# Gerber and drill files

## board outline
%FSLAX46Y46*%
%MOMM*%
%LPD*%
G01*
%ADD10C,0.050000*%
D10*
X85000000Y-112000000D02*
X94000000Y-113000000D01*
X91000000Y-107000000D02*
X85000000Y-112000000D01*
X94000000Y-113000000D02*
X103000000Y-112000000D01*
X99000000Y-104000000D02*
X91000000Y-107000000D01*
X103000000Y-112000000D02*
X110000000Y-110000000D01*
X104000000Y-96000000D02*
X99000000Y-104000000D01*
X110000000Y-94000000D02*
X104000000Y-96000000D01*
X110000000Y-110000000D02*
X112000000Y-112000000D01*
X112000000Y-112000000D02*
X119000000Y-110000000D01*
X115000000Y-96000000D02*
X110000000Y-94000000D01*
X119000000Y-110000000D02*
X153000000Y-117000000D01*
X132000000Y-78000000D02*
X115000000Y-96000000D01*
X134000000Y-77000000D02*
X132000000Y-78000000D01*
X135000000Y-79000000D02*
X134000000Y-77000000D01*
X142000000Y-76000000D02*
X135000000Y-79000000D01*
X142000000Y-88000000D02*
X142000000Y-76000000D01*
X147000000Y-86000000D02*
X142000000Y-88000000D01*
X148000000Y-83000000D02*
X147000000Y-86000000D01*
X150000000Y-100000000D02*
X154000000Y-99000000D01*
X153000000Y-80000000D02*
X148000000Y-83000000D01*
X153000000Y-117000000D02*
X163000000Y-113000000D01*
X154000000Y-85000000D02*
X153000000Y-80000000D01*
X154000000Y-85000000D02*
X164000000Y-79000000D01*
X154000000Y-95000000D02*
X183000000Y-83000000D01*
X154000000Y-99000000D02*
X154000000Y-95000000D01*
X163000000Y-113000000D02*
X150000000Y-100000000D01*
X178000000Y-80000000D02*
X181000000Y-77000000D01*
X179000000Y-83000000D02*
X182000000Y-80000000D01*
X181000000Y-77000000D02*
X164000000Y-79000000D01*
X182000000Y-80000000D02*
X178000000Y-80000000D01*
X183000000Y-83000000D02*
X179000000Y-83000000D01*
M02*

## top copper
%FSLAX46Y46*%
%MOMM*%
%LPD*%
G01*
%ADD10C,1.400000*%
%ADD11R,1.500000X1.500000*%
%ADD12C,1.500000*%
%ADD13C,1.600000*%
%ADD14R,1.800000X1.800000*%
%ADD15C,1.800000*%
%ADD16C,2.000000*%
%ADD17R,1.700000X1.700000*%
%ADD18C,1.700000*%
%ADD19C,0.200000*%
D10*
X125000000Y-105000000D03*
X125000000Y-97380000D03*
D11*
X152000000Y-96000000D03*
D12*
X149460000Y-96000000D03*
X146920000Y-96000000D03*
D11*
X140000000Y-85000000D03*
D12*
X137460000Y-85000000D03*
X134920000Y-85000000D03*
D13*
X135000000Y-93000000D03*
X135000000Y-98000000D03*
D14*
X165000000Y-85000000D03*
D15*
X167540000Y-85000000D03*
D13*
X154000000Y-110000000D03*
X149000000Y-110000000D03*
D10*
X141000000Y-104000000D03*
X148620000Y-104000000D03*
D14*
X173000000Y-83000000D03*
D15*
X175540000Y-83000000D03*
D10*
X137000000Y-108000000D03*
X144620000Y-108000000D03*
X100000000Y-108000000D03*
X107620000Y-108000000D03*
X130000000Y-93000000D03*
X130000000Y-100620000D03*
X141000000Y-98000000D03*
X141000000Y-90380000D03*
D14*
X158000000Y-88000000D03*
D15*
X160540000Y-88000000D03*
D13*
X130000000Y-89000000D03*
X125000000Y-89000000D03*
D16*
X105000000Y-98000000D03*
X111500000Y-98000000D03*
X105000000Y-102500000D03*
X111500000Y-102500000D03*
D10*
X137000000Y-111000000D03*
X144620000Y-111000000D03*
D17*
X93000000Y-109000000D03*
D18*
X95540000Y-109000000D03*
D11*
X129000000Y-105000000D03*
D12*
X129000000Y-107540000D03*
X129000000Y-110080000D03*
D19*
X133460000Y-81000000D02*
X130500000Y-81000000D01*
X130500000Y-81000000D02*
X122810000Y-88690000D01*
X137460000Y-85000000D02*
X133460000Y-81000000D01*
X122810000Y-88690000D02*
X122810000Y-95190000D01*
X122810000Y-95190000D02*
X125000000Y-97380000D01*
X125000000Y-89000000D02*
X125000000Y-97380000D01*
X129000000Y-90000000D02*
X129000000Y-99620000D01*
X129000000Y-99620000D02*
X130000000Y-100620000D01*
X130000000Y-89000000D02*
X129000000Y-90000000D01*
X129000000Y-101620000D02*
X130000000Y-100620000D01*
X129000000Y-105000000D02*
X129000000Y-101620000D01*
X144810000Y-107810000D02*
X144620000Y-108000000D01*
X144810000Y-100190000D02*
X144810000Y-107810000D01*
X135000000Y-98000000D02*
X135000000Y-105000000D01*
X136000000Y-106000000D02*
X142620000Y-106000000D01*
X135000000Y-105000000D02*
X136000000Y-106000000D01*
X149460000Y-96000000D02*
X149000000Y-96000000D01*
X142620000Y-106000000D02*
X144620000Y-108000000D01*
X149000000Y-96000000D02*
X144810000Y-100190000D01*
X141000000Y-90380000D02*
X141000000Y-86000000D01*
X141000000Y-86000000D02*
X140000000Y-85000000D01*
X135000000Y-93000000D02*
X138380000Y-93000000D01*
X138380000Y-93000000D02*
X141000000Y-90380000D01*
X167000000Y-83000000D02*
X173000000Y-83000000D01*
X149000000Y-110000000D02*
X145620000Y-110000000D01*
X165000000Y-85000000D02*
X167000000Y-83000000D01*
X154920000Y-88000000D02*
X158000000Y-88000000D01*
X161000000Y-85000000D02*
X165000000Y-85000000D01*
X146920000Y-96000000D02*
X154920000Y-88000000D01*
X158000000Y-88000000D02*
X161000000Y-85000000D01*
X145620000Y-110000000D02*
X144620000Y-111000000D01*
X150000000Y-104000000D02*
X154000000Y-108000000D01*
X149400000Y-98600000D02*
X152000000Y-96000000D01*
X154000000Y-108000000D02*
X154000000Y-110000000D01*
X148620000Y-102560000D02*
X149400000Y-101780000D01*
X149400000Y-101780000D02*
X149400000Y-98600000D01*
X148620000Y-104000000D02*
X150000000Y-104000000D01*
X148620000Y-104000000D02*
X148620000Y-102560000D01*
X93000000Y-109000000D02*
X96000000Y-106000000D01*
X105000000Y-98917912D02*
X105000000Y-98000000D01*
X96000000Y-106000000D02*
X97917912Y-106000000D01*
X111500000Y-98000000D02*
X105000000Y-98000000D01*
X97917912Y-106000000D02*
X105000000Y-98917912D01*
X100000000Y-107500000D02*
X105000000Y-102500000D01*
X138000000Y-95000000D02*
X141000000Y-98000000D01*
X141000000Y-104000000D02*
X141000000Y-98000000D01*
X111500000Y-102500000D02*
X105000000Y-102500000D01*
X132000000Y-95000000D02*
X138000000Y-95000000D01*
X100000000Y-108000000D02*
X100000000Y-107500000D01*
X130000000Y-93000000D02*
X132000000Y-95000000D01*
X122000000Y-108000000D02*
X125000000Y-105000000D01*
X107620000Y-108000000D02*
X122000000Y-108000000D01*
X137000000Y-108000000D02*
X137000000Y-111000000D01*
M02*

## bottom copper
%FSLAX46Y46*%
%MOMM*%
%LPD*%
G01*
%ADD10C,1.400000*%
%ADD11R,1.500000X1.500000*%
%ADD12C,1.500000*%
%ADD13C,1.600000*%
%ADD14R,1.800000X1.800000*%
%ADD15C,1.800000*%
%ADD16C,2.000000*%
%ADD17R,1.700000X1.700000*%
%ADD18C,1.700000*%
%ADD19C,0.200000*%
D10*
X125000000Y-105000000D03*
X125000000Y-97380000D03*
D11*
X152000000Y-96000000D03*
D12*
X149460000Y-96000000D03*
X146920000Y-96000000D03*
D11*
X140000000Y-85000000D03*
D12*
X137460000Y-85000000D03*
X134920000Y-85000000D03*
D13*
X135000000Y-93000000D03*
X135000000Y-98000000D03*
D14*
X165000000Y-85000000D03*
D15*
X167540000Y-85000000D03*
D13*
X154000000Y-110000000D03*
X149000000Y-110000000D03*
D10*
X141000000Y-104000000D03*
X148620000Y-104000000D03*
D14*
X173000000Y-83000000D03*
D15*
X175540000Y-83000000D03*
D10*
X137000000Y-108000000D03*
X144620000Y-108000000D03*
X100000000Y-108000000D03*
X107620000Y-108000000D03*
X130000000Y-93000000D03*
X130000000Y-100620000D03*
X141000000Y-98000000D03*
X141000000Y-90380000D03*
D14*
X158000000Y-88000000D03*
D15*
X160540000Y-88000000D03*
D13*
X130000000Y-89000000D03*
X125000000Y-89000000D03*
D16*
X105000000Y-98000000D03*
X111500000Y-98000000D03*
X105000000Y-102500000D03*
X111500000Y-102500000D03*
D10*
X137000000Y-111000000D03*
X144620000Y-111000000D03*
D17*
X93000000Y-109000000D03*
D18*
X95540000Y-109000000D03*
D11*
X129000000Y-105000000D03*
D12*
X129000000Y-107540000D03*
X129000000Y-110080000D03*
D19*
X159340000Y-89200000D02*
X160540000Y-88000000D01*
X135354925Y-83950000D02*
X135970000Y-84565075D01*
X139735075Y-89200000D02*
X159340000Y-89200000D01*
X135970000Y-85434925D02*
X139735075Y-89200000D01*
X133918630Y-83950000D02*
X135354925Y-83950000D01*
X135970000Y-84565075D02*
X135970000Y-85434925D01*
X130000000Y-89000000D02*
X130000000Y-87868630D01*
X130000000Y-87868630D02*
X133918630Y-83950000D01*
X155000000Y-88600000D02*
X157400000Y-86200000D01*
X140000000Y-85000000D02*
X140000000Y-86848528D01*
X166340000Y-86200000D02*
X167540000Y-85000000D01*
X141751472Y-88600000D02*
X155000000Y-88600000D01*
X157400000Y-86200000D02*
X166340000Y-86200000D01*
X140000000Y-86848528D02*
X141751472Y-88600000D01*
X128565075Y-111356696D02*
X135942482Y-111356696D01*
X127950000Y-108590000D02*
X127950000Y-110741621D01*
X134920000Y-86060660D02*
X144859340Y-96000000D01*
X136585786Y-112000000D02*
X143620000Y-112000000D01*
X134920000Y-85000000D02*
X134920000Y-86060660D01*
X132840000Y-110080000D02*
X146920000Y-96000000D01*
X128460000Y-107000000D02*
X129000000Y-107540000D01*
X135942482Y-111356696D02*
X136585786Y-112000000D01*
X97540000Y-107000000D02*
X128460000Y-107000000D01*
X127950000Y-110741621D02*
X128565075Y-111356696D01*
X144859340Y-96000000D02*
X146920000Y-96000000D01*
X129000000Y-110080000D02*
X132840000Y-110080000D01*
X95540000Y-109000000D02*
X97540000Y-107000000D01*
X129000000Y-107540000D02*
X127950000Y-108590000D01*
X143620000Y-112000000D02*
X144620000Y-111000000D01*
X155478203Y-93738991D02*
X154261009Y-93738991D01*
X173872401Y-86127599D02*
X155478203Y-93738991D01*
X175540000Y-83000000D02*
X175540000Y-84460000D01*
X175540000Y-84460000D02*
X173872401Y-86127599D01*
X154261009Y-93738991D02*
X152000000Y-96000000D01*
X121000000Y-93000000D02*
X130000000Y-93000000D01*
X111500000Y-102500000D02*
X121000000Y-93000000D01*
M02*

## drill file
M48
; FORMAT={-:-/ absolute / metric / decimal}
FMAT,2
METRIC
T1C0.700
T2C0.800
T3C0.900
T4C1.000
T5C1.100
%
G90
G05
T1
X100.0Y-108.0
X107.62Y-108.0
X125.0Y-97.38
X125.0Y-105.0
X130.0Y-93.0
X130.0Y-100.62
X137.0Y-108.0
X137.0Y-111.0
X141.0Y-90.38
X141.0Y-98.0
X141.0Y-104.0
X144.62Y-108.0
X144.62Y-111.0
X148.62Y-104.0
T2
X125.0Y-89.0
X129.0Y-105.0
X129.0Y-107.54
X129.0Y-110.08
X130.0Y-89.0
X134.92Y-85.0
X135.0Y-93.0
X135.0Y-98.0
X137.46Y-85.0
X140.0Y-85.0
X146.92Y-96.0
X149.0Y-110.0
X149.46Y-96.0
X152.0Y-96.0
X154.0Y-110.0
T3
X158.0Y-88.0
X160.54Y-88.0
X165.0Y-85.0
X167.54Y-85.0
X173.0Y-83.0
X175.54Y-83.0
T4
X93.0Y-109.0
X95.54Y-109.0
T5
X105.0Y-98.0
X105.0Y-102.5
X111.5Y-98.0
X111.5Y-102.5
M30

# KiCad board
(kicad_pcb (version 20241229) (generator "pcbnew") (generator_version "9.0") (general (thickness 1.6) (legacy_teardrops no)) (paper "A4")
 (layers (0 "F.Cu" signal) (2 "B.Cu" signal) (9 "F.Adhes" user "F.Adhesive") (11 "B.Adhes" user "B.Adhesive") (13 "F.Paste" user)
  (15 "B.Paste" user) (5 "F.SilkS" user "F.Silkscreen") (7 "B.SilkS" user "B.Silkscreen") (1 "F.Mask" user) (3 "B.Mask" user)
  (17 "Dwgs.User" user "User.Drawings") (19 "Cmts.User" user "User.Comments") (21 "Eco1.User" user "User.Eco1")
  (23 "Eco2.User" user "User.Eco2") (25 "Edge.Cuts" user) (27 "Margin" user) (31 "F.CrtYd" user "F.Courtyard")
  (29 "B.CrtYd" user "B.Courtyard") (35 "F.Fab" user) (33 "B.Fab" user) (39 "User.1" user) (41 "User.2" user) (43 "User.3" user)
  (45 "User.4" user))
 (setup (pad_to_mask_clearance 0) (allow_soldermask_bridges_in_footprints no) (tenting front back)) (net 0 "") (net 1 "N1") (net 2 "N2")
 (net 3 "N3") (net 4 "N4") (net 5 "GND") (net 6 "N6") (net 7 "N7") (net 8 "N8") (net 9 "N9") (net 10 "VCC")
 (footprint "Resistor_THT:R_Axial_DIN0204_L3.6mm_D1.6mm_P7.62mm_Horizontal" (layer "F.Cu") (at 125 105 90)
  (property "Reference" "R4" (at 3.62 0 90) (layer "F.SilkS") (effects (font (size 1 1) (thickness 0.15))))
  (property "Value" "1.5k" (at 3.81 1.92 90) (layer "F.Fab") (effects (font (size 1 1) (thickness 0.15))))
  (pad "1" thru_hole circle (at 0 0 90) (size 1.4 1.4) (drill 0.7) (layers "*.Cu" "*.Mask") (remove_unused_layers no) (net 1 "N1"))
  (pad "2" thru_hole circle (at 7.62 0 90) (size 1.4 1.4) (drill 0.7) (layers "*.Cu" "*.Mask") (remove_unused_layers no) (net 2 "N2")))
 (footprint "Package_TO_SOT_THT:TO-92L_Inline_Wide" (layer "F.Cu") (at 152 96 180)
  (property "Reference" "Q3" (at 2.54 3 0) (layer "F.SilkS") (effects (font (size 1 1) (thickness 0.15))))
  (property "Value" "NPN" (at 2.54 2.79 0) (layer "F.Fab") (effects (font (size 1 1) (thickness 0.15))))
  (pad "1" thru_hole rect (at 0 0 180) (size 1.5 1.5) (drill 0.8) (layers "*.Cu" "*.Mask") (remove_unused_layers no) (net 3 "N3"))
  (pad "2" thru_hole circle (at 2.54 0 180) (size 1.5 1.5) (drill 0.8) (layers "*.Cu" "*.Mask") (remove_unused_layers no) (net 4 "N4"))
  (pad "3" thru_hole circle (at 5.08 0 180) (size 1.5 1.5) (drill 0.8) (layers "*.Cu" "*.Mask") (remove_unused_layers no) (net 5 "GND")))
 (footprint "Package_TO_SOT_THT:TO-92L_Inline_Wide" (layer "F.Cu") (at 140 85 180)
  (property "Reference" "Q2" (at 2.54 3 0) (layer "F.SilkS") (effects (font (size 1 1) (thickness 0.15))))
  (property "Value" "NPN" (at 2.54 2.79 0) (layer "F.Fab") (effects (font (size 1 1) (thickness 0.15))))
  (pad "1" thru_hole rect (at 0 0 180) (size 1.5 1.5) (drill 0.8) (layers "*.Cu" "*.Mask") (remove_unused_layers no) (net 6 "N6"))
  (pad "2" thru_hole circle (at 2.54 0 180) (size 1.5 1.5) (drill 0.8) (layers "*.Cu" "*.Mask") (remove_unused_layers no) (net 2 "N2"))
  (pad "3" thru_hole circle (at 5.08 0 180) (size 1.5 1.5) (drill 0.8) (layers "*.Cu" "*.Mask") (remove_unused_layers no) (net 5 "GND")))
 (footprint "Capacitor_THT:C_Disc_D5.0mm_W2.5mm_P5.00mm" (layer "F.Cu") (at 135 93 -90)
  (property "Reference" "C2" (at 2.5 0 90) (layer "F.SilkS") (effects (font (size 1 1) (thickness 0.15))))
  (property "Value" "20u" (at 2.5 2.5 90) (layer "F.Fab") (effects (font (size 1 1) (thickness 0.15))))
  (pad "1" thru_hole circle (at 0 0 270) (size 1.6 1.6) (drill 0.8) (layers "*.Cu" "*.Mask") (remove_unused_layers no) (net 6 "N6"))
  (pad "2" thru_hole circle (at 5 0 270) (size 1.6 1.6) (drill 0.8) (layers "*.Cu" "*.Mask") (remove_unused_layers no) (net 4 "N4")))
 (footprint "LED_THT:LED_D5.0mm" (layer "F.Cu") (at 165 85)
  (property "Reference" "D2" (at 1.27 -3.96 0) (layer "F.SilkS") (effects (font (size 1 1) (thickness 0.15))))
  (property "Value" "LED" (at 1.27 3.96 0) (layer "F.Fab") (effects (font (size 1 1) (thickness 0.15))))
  (pad "1" thru_hole rect (at 0 0) (size 1.8 1.8) (drill 0.9) (layers "*.Cu" "*.Mask") (remove_unused_layers no) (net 5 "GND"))
  (pad "2" thru_hole circle (at 2.54 0) (size 1.8 1.8) (drill 0.9) (layers "*.Cu" "*.Mask") (remove_unused_layers no) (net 6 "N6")))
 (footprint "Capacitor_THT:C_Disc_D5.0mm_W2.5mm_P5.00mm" (layer "F.Cu") (at 154 110 180)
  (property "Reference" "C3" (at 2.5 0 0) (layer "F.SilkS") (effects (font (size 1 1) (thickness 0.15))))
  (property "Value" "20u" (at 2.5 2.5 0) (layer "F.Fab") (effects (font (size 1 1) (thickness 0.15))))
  (pad "1" thru_hole circle (at 0 0 180) (size 1.6 1.6) (drill 0.8) (layers "*.Cu" "*.Mask") (remove_unused_layers no) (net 3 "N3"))
  (pad "2" thru_hole circle (at 5 0 180) (size 1.6 1.6) (drill 0.8) (layers "*.Cu" "*.Mask") (remove_unused_layers no) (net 5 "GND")))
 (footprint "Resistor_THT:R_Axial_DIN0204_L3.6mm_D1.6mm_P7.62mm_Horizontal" (layer "F.Cu") (at 141 104)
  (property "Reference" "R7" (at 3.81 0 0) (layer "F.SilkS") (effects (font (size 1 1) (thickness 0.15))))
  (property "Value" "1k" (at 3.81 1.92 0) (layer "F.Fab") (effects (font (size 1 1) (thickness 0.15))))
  (pad "1" thru_hole circle (at 0 0) (size 1.4 1.4) (drill 0.7) (layers "*.Cu" "*.Mask") (remove_unused_layers no) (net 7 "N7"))
  (pad "2" thru_hole circle (at 7.62 0) (size 1.4 1.4) (drill 0.7) (layers "*.Cu" "*.Mask") (remove_unused_layers no) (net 3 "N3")))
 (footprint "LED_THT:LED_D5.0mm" (layer "F.Cu") (at 173 83)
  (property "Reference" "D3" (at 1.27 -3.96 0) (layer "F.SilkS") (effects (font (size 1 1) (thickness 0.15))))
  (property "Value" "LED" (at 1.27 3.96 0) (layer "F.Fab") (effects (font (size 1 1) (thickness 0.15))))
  (pad "1" thru_hole rect (at 0 0) (size 1.8 1.8) (drill 0.9) (layers "*.Cu" "*.Mask") (remove_unused_layers no) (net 5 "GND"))
  (pad "2" thru_hole circle (at 2.54 0) (size 1.8 1.8) (drill 0.9) (layers "*.Cu" "*.Mask") (remove_unused_layers no) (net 3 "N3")))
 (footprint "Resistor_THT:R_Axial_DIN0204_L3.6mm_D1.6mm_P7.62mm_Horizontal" (layer "F.Cu") (at 137 108)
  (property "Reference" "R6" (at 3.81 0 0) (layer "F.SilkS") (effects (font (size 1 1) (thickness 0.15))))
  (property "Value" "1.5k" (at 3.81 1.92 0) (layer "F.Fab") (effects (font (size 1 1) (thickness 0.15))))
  (pad "1" thru_hole circle (at 0 0) (size 1.4 1.4) (drill 0.7) (layers "*.Cu" "*.Mask") (remove_unused_layers no) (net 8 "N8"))
  (pad "2" thru_hole circle (at 7.62 0) (size 1.4 1.4) (drill 0.7) (layers "*.Cu" "*.Mask") (remove_unused_layers no) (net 4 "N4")))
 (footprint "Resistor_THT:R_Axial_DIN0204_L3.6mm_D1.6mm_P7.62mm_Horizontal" (layer "F.Cu") (at 100 108)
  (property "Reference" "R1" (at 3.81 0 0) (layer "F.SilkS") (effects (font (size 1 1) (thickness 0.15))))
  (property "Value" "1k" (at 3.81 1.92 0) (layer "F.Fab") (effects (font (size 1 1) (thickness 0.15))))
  (pad "1" thru_hole circle (at 0 0) (size 1.4 1.4) (drill 0.7) (layers "*.Cu" "*.Mask") (remove_unused_layers no) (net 7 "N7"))
  (pad "2" thru_hole circle (at 7.62 0) (size 1.4 1.4) (drill 0.7) (layers "*.Cu" "*.Mask") (remove_unused_layers no) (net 1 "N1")))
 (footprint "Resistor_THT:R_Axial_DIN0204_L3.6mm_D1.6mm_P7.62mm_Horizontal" (layer "F.Cu") (at 130 93 -90)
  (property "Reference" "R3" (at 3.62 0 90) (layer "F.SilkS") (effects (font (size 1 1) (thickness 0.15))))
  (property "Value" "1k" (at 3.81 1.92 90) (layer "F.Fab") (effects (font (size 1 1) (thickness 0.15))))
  (pad "1" thru_hole circle (at 0 0 270) (size 1.4 1.4) (drill 0.7) (layers "*.Cu" "*.Mask") (remove_unused_layers no) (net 7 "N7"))
  (pad "2" thru_hole circle (at 7.62 0 270) (size 1.4 1.4) (drill 0.7) (layers "*.Cu" "*.Mask") (remove_unused_layers no) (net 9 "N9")))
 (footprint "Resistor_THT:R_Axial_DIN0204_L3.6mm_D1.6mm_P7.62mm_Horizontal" (layer "F.Cu") (at 141 98 90)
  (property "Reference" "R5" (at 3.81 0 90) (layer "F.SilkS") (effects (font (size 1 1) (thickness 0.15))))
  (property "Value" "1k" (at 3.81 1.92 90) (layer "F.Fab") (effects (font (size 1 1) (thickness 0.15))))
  (pad "1" thru_hole circle (at 0 0 90) (size 1.4 1.4) (drill 0.7) (layers "*.Cu" "*.Mask") (remove_unused_layers no) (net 7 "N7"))
  (pad "2" thru_hole circle (at 7.62 0 90) (size 1.4 1.4) (drill 0.7) (layers "*.Cu" "*.Mask") (remove_unused_layers no) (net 6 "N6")))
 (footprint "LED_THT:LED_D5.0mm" (layer "F.Cu") (at 158 88)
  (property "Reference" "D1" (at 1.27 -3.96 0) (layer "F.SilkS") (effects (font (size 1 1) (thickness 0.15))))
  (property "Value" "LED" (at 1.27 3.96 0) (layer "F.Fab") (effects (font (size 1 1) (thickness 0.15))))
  (pad "1" thru_hole rect (at 0 0) (size 1.8 1.8) (drill 0.9) (layers "*.Cu" "*.Mask") (remove_unused_layers no) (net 5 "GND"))
  (pad "2" thru_hole circle (at 2.54 0) (size 1.8 1.8) (drill 0.9) (layers "*.Cu" "*.Mask") (remove_unused_layers no) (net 9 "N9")))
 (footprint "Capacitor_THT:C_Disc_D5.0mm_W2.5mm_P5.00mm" (layer "F.Cu") (at 130 89 180)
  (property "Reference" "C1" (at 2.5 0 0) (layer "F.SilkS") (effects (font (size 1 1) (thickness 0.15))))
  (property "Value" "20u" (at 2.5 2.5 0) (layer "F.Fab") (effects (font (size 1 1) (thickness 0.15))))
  (pad "1" thru_hole circle (at 0 0 180) (size 1.6 1.6) (drill 0.8) (layers "*.Cu" "*.Mask") (remove_unused_layers no) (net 9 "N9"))
  (pad "2" thru_hole circle (at 5 0 180) (size 1.6 1.6) (drill 0.8) (layers "*.Cu" "*.Mask") (remove_unused_layers no) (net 2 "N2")))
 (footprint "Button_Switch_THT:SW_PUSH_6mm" (layer "F.Cu") (at 105 98)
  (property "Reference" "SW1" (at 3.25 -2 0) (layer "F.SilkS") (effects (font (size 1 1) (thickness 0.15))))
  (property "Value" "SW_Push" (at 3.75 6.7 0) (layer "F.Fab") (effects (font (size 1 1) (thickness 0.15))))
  (pad "1" thru_hole circle (at 0 0 90) (size 2 2) (drill 1.1) (layers "*.Cu" "*.Mask") (remove_unused_layers no) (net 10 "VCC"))
  (pad "1" thru_hole circle (at 6.5 0 90) (size 2 2) (drill 1.1) (layers "*.Cu" "*.Mask") (remove_unused_layers no) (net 10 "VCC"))
  (pad "2" thru_hole circle (at 0 4.5 90) (size 2 2) (drill 1.1) (layers "*.Cu" "*.Mask") (remove_unused_layers no) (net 7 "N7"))
  (pad "2" thru_hole circle (at 6.5 4.5 90) (size 2 2) (drill 1.1) (layers "*.Cu" "*.Mask") (remove_unused_layers no) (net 7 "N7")))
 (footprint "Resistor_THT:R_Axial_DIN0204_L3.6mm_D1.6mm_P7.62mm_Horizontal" (layer "F.Cu") (at 137 111)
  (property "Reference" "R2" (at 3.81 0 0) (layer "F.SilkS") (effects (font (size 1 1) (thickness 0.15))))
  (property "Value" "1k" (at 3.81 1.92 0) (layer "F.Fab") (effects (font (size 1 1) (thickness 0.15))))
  (pad "1" thru_hole circle (at 0 0) (size 1.4 1.4) (drill 0.7) (layers "*.Cu" "*.Mask") (remove_unused_layers no) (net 8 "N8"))
  (pad "2" thru_hole circle (at 7.62 0) (size 1.4 1.4) (drill 0.7) (layers "*.Cu" "*.Mask") (remove_unused_layers no) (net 5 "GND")))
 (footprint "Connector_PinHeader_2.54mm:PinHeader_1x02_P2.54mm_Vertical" (layer "F.Cu") (at 93 109 90)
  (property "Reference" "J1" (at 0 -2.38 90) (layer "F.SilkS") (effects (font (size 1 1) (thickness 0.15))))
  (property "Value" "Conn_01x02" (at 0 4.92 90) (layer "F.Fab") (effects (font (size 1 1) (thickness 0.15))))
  (pad "1" thru_hole rect (at 0 0 90) (size 1.7 1.7) (drill 1) (layers "*.Cu" "*.Mask") (remove_unused_layers no) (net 10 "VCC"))
  (pad "2" thru_hole circle (at 0 2.54 90) (size 1.7 1.7) (drill 1) (layers "*.Cu" "*.Mask") (remove_unused_layers no) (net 5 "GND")))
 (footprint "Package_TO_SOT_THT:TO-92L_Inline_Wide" (layer "F.Cu") (at 129 105 -90)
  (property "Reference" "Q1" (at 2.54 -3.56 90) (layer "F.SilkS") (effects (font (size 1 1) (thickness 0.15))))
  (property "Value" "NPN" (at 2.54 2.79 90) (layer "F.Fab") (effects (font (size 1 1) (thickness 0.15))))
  (pad "1" thru_hole rect (at 0 0 270) (size 1.5 1.5) (drill 0.8) (layers "*.Cu" "*.Mask") (remove_unused_layers no) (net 9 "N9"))
  (pad "2" thru_hole circle (at 2.54 0 270) (size 1.5 1.5) (drill 0.8) (layers "*.Cu" "*.Mask") (remove_unused_layers no) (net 5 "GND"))
  (pad "3" thru_hole circle (at 5.08 0 270) (size 1.5 1.5) (drill 0.8) (layers "*.Cu" "*.Mask") (remove_unused_layers no) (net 5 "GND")))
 (gr_line (start 85 112) (end 94 113) (stroke (width 0.05) (type default)) (layer "Edge.Cuts"))
 (gr_line (start 91 107) (end 85 112) (stroke (width 0.05) (type default)) (layer "Edge.Cuts"))
 (gr_line (start 94 113) (end 103 112) (stroke (width 0.05) (type default)) (layer "Edge.Cuts"))
 (gr_line (start 99 104) (end 91 107) (stroke (width 0.05) (type default)) (layer "Edge.Cuts"))
 (gr_line (start 103 112) (end 110 110) (stroke (width 0.05) (type default)) (layer "Edge.Cuts"))
 (gr_line (start 104 96) (end 99 104) (stroke (width 0.05) (type default)) (layer "Edge.Cuts"))
 (gr_line (start 110 94) (end 104 96) (stroke (width 0.05) (type default)) (layer "Edge.Cuts"))
 (gr_line (start 110 110) (end 112 112) (stroke (width 0.05) (type default)) (layer "Edge.Cuts"))
 (gr_line (start 112 112) (end 119 110) (stroke (width 0.05) (type default)) (layer "Edge.Cuts"))
 (gr_line (start 115 96) (end 110 94) (stroke (width 0.05) (type default)) (layer "Edge.Cuts"))
 (gr_line (start 119 110) (end 153 117) (stroke (width 0.05) (type default)) (layer "Edge.Cuts"))
 (gr_line (start 132 78) (end 115 96) (stroke (width 0.05) (type default)) (layer "Edge.Cuts"))
 (gr_line (start 134 77) (end 132 78) (stroke (width 0.05) (type default)) (layer "Edge.Cuts"))
 (gr_line (start 135 79) (end 134 77) (stroke (width 0.05) (type default)) (layer "Edge.Cuts"))
 (gr_line (start 142 76) (end 135 79) (stroke (width 0.05) (type default)) (layer "Edge.Cuts"))
 (gr_line (start 142 88) (end 142 76) (stroke (width 0.05) (type default)) (layer "Edge.Cuts"))
 (gr_line (start 147 86) (end 142 88) (stroke (width 0.05) (type default)) (layer "Edge.Cuts"))
 (gr_line (start 148 83) (end 147 86) (stroke (width 0.05) (type default)) (layer "Edge.Cuts"))
 (gr_line (start 150 100) (end 154 99) (stroke (width 0.05) (type default)) (layer "Edge.Cuts"))
 (gr_line (start 153 80) (end 148 83) (stroke (width 0.05) (type default)) (layer "Edge.Cuts"))
 (gr_line (start 153 117) (end 163 113) (stroke (width 0.05) (type default)) (layer "Edge.Cuts"))
 (gr_line (start 154 85) (end 153 80) (stroke (width 0.05) (type default)) (layer "Edge.Cuts"))
 (gr_line (start 154 85) (end 164 79) (stroke (width 0.05) (type default)) (layer "Edge.Cuts"))
 (gr_line (start 154 95) (end 183 83) (stroke (width 0.05) (type default)) (layer "Edge.Cuts"))
 (gr_line (start 154 99) (end 154 95) (stroke (width 0.05) (type default)) (layer "Edge.Cuts"))
 (gr_line (start 163 113) (end 150 100) (stroke (width 0.05) (type default)) (layer "Edge.Cuts"))
 (gr_line (start 178 80) (end 181 77) (stroke (width 0.05) (type default)) (layer "Edge.Cuts"))
 (gr_line (start 179 83) (end 182 80) (stroke (width 0.05) (type default)) (layer "Edge.Cuts"))
 (gr_line (start 181 77) (end 164 79) (stroke (width 0.05) (type default)) (layer "Edge.Cuts"))
 (gr_line (start 182 80) (end 178 80) (stroke (width 0.05) (type default)) (layer "Edge.Cuts"))
 (gr_line (start 183 83) (end 179 83) (stroke (width 0.05) (type default)) (layer "Edge.Cuts"))
 (segment (start 133.46 81) (end 130.5 81) (width 0.2) (layer "F.Cu") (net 2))
 (segment (start 130.5 81) (end 122.81 88.69) (width 0.2) (layer "F.Cu") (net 2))
 (segment (start 137.46 85) (end 133.46 81) (width 0.2) (layer "F.Cu") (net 2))
 (segment (start 122.81 88.69) (end 122.81 95.19) (width 0.2) (layer "F.Cu") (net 2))
 (segment (start 122.81 95.19) (end 125 97.38) (width 0.2) (layer "F.Cu") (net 2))
 (segment (start 125 89) (end 125 97.38) (width 0.2) (layer "F.Cu") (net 2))
 (segment (start 129 90) (end 129 99.62) (width 0.2) (layer "F.Cu") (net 9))
 (segment (start 129 99.62) (end 130 100.62) (width 0.2) (layer "F.Cu") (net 9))
 (segment (start 130 89) (end 129 90) (width 0.2) (layer "F.Cu") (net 9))
 (segment (start 129 101.62) (end 130 100.62) (width 0.2) (layer "F.Cu") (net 9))
 (segment (start 129 105) (end 129 101.62) (width 0.2) (layer "F.Cu") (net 9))
 (segment (start 159.34 89.2) (end 160.54 88) (width 0.2) (layer "B.Cu") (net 9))
 (segment (start 135.354925 83.95) (end 135.97 84.565075) (width 0.2) (layer "B.Cu") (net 9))
 (segment (start 139.735075 89.2) (end 159.34 89.2) (width 0.2) (layer "B.Cu") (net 9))
 (segment (start 135.97 85.434925) (end 139.735075 89.2) (width 0.2) (layer "B.Cu") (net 9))
 (segment (start 133.91863 83.95) (end 135.354925 83.95) (width 0.2) (layer "B.Cu") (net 9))
 (segment (start 135.97 84.565075) (end 135.97 85.434925) (width 0.2) (layer "B.Cu") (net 9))
 (segment (start 130 89) (end 130 87.86863) (width 0.2) (layer "B.Cu") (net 9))
 (segment (start 130 87.86863) (end 133.91863 83.95) (width 0.2) (layer "B.Cu") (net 9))
 (segment (start 144.81 107.81) (end 144.62 108) (width 0.2) (layer "F.Cu") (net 4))
 (segment (start 144.81 100.19) (end 144.81 107.81) (width 0.2) (layer "F.Cu") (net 4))
 (segment (start 135 98) (end 135 105) (width 0.2) (layer "F.Cu") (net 4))
 (segment (start 136 106) (end 142.62 106) (width 0.2) (layer "F.Cu") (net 4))
 (segment (start 135 105) (end 136 106) (width 0.2) (layer "F.Cu") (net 4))
 (segment (start 149.46 96) (end 149 96) (width 0.2) (layer "F.Cu") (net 4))
 (segment (start 142.62 106) (end 144.62 108) (width 0.2) (layer "F.Cu") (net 4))
 (segment (start 149 96) (end 144.81 100.19) (width 0.2) (layer "F.Cu") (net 4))
 (segment (start 141 90.38) (end 141 86) (width 0.2) (layer "F.Cu") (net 6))
 (segment (start 141 86) (end 140 85) (width 0.2) (layer "F.Cu") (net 6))
 (segment (start 135 93) (end 138.38 93) (width 0.2) (layer "F.Cu") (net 6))
 (segment (start 138.38 93) (end 141 90.38) (width 0.2) (layer "F.Cu") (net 6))
 (segment (start 155 88.6) (end 157.4 86.2) (width 0.2) (layer "B.Cu") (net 6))
 (segment (start 140 85) (end 140 86.848528) (width 0.2) (layer "B.Cu") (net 6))
 (segment (start 166.34 86.2) (end 167.54 85) (width 0.2) (layer "B.Cu") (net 6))
 (segment (start 141.751472 88.6) (end 155 88.6) (width 0.2) (layer "B.Cu") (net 6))
 (segment (start 157.4 86.2) (end 166.34 86.2) (width 0.2) (layer "B.Cu") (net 6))
 (segment (start 140 86.848528) (end 141.751472 88.6) (width 0.2) (layer "B.Cu") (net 6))
 (segment (start 167 83) (end 173 83) (width 0.2) (layer "F.Cu") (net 5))
 (segment (start 149 110) (end 145.62 110) (width 0.2) (layer "F.Cu") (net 5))
 (segment (start 165 85) (end 167 83) (width 0.2) (layer "F.Cu") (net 5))
 (segment (start 154.92 88) (end 158 88) (width 0.2) (layer "F.Cu") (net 5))
 (segment (start 161 85) (end 165 85) (width 0.2) (layer "F.Cu") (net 5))
 (segment (start 146.92 96) (end 154.92 88) (width 0.2) (layer "F.Cu") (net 5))
 (segment (start 158 88) (end 161 85) (width 0.2) (layer "F.Cu") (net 5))
 (segment (start 145.62 110) (end 144.62 111) (width 0.2) (layer "F.Cu") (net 5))
 (segment (start 128.565075 111.356696) (end 135.942482 111.356696) (width 0.2) (layer "B.Cu") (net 5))
 (segment (start 127.95 108.59) (end 127.95 110.741621) (width 0.2) (layer "B.Cu") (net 5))
 (segment (start 134.92 86.06066) (end 144.85934 96) (width 0.2) (layer "B.Cu") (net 5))
 (segment (start 136.585786 112) (end 143.62 112) (width 0.2) (layer "B.Cu") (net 5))
 (segment (start 134.92 85) (end 134.92 86.06066) (width 0.2) (layer "B.Cu") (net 5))
 (segment (start 132.84 110.08) (end 146.92 96) (width 0.2) (layer "B.Cu") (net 5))
 (segment (start 128.46 107) (end 129 107.54) (width 0.2) (layer "B.Cu") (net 5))
 (segment (start 135.942482 111.356696) (end 136.585786 112) (width 0.2) (layer "B.Cu") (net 5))
 (segment (start 97.54 107) (end 128.46 107) (width 0.2) (layer "B.Cu") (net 5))
 (segment (start 127.95 110.741621) (end 128.565075 111.356696) (width 0.2) (layer "B.Cu") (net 5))
 (segment (start 144.85934 96) (end 146.92 96) (width 0.2) (layer "B.Cu") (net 5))
 (segment (start 129 110.08) (end 132.84 110.08) (width 0.2) (layer "B.Cu") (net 5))
 (segment (start 95.54 109) (end 97.54 107) (width 0.2) (layer "B.Cu") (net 5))
 (segment (start 129 107.54) (end 127.95 108.59) (width 0.2) (layer "B.Cu") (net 5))
 (segment (start 143.62 112) (end 144.62 111) (width 0.2) (layer "B.Cu") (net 5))
 (segment (start 150 104) (end 154 108) (width 0.2) (layer "F.Cu") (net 3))
 (segment (start 149.4 98.6) (end 152 96) (width 0.2) (layer "F.Cu") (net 3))
 (segment (start 154 108) (end 154 110) (width 0.2) (layer "F.Cu") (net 3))
 (segment (start 148.62 102.56) (end 149.4 101.78) (width 0.2) (layer "F.Cu") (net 3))
 (segment (start 149.4 101.78) (end 149.4 98.6) (width 0.2) (layer "F.Cu") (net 3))
 (segment (start 148.62 104) (end 150 104) (width 0.2) (layer "F.Cu") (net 3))
 (segment (start 148.62 104) (end 148.62 102.56) (width 0.2) (layer "F.Cu") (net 3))
 (segment (start 155.478203 93.738991) (end 154.261009 93.738991) (width 0.2) (layer "B.Cu") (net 3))
 (segment (start 173.872401 86.127599) (end 155.478203 93.738991) (width 0.2) (layer "B.Cu") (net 3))
 (segment (start 175.54 83) (end 175.54 84.46) (width 0.2) (layer "B.Cu") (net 3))
 (segment (start 175.54 84.46) (end 173.872401 86.127599) (width 0.2) (layer "B.Cu") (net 3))
 (segment (start 154.261009 93.738991) (end 152 96) (width 0.2) (layer "B.Cu") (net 3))
 (segment (start 93 109) (end 96 106) (width 0.2) (layer "F.Cu") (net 10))
 (segment (start 105 98.917912) (end 105 98) (width 0.2) (layer "F.Cu") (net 10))
 (segment (start 96 106) (end 97.917912 106) (width 0.2) (layer "F.Cu") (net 10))
 (segment (start 111.5 98) (end 105 98) (width 0.2) (layer "F.Cu") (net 10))
 (segment (start 97.917912 106) (end 105 98.917912) (width 0.2) (layer "F.Cu") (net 10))
 (segment (start 100 107.5) (end 105 102.5) (width 0.2) (layer "F.Cu") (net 7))
 (segment (start 138 95) (end 141 98) (width 0.2) (layer "F.Cu") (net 7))
 (segment (start 141 104) (end 141 98) (width 0.2) (layer "F.Cu") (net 7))
 (segment (start 111.5 102.5) (end 105 102.5) (width 0.2) (layer "F.Cu") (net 7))
 (segment (start 132 95) (end 138 95) (width 0.2) (layer "F.Cu") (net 7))
 (segment (start 100 108) (end 100 107.5) (width 0.2) (layer "F.Cu") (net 7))
 (segment (start 130 93) (end 132 95) (width 0.2) (layer "F.Cu") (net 7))
 (segment (start 121 93) (end 130 93) (width 0.2) (layer "B.Cu") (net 7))
 (segment (start 111.5 102.5) (end 121 93) (width 0.2) (layer "B.Cu") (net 7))
 (segment (start 122 108) (end 125 105) (width 0.2) (layer "F.Cu") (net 1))
 (segment (start 107.62 108) (end 122 108) (width 0.2) (layer "F.Cu") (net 1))
 (segment (start 137 108) (end 137 111) (width 0.2) (layer "F.Cu") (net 8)))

